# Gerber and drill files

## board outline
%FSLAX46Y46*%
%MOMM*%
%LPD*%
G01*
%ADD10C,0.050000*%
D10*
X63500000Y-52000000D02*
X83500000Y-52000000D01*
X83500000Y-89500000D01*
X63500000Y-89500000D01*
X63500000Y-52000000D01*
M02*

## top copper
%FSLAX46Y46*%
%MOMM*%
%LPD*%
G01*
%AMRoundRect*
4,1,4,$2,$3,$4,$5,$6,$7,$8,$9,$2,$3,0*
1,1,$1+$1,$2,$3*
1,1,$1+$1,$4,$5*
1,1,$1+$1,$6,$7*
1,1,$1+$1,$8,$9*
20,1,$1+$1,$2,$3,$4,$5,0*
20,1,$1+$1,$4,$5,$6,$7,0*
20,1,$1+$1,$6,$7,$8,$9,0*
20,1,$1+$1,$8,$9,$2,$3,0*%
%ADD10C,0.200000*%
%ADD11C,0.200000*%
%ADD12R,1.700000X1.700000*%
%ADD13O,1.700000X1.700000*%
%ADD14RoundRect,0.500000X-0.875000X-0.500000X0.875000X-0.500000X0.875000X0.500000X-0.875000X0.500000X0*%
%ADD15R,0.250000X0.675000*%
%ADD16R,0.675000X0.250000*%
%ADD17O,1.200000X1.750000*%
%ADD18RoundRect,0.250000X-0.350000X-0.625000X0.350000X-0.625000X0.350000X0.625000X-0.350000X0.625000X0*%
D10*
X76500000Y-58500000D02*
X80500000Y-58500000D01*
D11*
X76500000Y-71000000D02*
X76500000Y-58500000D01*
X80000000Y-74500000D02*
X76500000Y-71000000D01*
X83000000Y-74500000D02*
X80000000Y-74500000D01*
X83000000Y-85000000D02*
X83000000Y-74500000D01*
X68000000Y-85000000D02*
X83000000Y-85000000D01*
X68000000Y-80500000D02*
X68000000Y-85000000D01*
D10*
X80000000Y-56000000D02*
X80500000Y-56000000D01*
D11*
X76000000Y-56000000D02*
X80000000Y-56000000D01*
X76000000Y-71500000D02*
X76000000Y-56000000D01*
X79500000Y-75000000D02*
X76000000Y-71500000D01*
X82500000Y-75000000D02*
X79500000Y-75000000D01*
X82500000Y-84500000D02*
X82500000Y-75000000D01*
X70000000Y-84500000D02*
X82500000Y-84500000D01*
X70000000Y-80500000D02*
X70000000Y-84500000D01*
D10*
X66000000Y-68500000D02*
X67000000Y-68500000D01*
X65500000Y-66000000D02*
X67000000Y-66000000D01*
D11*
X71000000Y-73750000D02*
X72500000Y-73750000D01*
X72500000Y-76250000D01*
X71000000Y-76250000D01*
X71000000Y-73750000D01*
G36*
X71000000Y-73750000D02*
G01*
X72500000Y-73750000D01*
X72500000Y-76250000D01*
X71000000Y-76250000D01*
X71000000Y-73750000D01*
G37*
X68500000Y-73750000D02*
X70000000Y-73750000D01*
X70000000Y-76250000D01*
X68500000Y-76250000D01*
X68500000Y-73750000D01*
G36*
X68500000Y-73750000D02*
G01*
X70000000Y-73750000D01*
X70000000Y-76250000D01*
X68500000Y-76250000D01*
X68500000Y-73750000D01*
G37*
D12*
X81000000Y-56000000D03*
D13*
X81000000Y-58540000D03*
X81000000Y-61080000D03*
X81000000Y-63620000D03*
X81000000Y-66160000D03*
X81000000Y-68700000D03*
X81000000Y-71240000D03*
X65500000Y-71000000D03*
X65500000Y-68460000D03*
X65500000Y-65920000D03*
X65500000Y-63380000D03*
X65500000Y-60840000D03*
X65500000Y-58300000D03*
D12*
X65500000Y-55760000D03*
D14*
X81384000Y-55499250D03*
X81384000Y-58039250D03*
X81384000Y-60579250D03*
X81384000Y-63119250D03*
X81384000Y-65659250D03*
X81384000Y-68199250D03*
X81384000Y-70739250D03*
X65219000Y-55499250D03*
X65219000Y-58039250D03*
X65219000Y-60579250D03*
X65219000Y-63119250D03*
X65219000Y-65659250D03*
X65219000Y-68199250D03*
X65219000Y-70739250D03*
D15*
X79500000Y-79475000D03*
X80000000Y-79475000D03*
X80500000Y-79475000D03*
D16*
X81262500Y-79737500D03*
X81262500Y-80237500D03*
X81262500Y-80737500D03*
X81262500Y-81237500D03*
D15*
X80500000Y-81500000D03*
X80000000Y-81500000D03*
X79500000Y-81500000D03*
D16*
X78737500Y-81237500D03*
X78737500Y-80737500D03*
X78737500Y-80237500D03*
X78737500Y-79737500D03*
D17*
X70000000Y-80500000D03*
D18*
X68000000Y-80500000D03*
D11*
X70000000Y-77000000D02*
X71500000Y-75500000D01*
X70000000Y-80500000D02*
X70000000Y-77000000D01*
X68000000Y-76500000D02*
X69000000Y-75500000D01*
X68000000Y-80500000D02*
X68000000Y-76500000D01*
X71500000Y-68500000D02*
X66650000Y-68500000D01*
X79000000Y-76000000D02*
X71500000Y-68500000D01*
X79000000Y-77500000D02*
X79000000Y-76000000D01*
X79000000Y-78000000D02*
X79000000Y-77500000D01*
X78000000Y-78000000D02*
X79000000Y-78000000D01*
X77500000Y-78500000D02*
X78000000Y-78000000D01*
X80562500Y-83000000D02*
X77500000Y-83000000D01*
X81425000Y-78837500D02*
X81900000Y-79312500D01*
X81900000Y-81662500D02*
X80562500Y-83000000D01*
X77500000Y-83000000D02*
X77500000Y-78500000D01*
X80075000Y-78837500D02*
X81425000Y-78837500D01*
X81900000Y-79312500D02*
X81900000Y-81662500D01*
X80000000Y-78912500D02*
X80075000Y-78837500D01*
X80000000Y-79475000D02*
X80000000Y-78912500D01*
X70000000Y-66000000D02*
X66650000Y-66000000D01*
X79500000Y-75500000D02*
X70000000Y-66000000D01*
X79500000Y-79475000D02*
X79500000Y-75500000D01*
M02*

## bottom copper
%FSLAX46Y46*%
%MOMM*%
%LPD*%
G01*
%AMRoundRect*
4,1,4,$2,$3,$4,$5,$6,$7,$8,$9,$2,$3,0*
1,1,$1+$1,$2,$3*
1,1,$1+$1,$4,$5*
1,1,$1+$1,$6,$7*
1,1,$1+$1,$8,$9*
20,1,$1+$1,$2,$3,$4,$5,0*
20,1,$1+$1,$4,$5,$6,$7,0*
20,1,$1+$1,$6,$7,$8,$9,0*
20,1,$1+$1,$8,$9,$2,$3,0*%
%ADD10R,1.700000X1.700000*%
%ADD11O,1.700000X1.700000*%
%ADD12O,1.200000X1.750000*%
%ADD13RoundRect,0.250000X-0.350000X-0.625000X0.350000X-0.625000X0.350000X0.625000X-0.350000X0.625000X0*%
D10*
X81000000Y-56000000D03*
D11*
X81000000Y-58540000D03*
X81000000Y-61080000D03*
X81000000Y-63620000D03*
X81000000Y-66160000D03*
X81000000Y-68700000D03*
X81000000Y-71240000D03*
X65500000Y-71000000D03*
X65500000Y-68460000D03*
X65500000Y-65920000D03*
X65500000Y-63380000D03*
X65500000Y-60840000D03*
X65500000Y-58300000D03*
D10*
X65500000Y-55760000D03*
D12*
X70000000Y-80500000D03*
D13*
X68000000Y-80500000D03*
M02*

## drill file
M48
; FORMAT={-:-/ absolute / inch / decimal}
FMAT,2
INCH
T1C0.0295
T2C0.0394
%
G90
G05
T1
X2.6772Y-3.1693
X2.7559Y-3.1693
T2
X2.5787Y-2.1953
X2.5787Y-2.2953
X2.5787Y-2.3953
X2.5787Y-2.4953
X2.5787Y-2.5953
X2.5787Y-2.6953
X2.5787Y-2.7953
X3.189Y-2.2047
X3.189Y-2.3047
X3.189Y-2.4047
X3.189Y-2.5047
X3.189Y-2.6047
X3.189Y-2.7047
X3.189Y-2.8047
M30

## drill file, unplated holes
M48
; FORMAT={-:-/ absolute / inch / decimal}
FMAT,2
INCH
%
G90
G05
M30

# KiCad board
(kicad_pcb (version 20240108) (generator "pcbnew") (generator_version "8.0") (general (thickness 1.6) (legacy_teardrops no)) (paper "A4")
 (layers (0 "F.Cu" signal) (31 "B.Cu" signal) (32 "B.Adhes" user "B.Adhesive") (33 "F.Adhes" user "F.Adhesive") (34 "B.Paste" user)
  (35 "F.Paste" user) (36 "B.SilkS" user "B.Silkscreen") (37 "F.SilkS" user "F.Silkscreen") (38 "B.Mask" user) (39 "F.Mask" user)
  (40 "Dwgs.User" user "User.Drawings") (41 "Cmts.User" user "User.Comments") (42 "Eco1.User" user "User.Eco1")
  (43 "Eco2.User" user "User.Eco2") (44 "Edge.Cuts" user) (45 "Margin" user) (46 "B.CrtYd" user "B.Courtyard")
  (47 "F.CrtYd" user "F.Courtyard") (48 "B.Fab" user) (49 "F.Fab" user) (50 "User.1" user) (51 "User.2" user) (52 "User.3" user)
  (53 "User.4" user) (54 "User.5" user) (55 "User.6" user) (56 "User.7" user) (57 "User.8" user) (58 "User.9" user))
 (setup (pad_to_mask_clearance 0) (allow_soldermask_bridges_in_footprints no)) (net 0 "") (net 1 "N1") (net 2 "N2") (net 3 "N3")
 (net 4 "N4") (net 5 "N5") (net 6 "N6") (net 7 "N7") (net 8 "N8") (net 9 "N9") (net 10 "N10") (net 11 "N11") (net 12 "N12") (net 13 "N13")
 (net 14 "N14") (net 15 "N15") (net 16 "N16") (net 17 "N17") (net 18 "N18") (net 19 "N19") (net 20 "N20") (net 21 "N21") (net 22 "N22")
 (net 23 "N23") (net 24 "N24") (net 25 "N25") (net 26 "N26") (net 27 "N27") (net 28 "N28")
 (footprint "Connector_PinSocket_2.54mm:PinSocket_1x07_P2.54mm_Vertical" (layer "F.Cu") (at 65.5 55.76)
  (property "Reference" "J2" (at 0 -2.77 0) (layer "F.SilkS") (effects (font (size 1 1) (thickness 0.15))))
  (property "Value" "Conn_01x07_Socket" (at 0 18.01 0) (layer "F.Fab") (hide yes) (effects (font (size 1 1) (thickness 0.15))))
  (pad "1" thru_hole rect (at 0 0) (size 1.7 1.7) (drill 1) (layers "*.Cu" "*.Mask") (remove_unused_layers no) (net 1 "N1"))
  (pad "2" thru_hole oval (at 0 2.54) (size 1.7 1.7) (drill 1) (layers "*.Cu" "*.Mask") (remove_unused_layers no) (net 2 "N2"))
  (pad "3" thru_hole oval (at 0 5.08) (size 1.7 1.7) (drill 1) (layers "*.Cu" "*.Mask") (remove_unused_layers no) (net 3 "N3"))
  (pad "4" thru_hole oval (at 0 7.62) (size 1.7 1.7) (drill 1) (layers "*.Cu" "*.Mask") (remove_unused_layers no) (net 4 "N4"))
  (pad "5" thru_hole oval (at 0 10.16) (size 1.7 1.7) (drill 1) (layers "*.Cu" "*.Mask") (remove_unused_layers no) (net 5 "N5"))
  (pad "6" thru_hole oval (at 0 12.7) (size 1.7 1.7) (drill 1) (layers "*.Cu" "*.Mask") (remove_unused_layers no) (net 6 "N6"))
  (pad "7" thru_hole oval (at 0 15.24) (size 1.7 1.7) (drill 1) (layers "*.Cu" "*.Mask") (remove_unused_layers no) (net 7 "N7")))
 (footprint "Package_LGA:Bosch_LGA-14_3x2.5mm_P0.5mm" (layer "F.Cu") (at 80 80.4875)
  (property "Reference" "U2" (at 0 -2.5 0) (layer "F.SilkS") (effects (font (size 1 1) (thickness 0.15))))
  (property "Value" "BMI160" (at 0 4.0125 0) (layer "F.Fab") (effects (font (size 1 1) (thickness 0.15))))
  (pad "1" smd rect (at -1.2625 -0.75) (size 0.675 0.25) (layers "F.Cu" "F.Paste" "F.Mask") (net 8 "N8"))
  (pad "2" smd rect (at -1.2625 -0.25) (size 0.675 0.25) (layers "F.Cu" "F.Paste" "F.Mask") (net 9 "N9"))
  (pad "3" smd rect (at -1.2625 0.25) (size 0.675 0.25) (layers "F.Cu" "F.Paste" "F.Mask") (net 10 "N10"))
  (pad "4" smd rect (at -1.2625 0.75) (size 0.675 0.25) (layers "F.Cu" "F.Paste" "F.Mask") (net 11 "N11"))
  (pad "5" smd rect (at -0.5 1.0125) (size 0.25 0.675) (layers "F.Cu" "F.Paste" "F.Mask") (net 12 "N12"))
  (pad "6" smd rect (at 0 1.0125) (size 0.25 0.675) (layers "F.Cu" "F.Paste" "F.Mask") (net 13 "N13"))
  (pad "7" smd rect (at 0.5 1.0125) (size 0.25 0.675) (layers "F.Cu" "F.Paste" "F.Mask") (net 13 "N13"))
  (pad "8" smd rect (at 1.2625 0.75) (size 0.675 0.25) (layers "F.Cu" "F.Paste" "F.Mask") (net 12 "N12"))
  (pad "9" smd rect (at 1.2625 0.25) (size 0.675 0.25) (layers "F.Cu" "F.Paste" "F.Mask") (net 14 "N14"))
  (pad "10" smd rect (at 1.2625 -0.25) (size 0.675 0.25) (layers "F.Cu" "F.Paste" "F.Mask") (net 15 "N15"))
  (pad "11" smd rect (at 1.2625 -0.75) (size 0.675 0.25) (layers "F.Cu" "F.Paste" "F.Mask") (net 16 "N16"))
  (pad "12" smd rect (at 0.5 -1.0125) (size 0.25 0.675) (layers "F.Cu" "F.Paste" "F.Mask") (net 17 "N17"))
  (pad "13" smd rect (at 0 -1.0125) (size 0.25 0.675) (layers "F.Cu" "F.Paste" "F.Mask") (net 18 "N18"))
  (pad "14" smd rect (at -0.5 -1.0125) (size 0.25 0.675) (layers "F.Cu" "F.Paste" "F.Mask") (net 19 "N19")))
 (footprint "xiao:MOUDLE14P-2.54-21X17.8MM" (layer "F.Cu") (at 64.384 73.61925)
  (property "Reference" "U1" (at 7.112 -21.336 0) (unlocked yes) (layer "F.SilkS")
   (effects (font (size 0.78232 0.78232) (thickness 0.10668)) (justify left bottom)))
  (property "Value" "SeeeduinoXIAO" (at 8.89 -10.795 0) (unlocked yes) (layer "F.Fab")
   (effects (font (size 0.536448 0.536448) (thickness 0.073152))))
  (pad "1" smd roundrect (at 0.835 -18.12) (size 2.75 2) (layers "F.Cu" "F.Paste" "F.Mask") (roundrect_rratio 0.25) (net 1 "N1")
   (solder_mask_margin 0.1016) (thermal_bridge_angle 0))
  (pad "2" smd roundrect (at 0.835 -15.58) (size 2.75 2) (layers "F.Cu" "F.Paste" "F.Mask") (roundrect_rratio 0.25) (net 2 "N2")
   (solder_mask_margin 0.1016) (thermal_bridge_angle 0))
  (pad "3" smd roundrect (at 0.835 -13.04) (size 2.75 2) (layers "F.Cu" "F.Paste" "F.Mask") (roundrect_rratio 0.25) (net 3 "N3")
   (solder_mask_margin 0.1016) (thermal_bridge_angle 0))
  (pad "4" smd roundrect (at 0.835 -10.5) (size 2.75 2) (layers "F.Cu" "F.Paste" "F.Mask") (roundrect_rratio 0.25) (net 4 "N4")
   (solder_mask_margin 0.1016) (thermal_bridge_angle 0))
  (pad "5" smd roundrect (at 0.835 -7.96) (size 2.75 2) (layers "F.Cu" "F.Paste" "F.Mask") (roundrect_rratio 0.25) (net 5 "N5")
   (solder_mask_margin 0.1016) (thermal_bridge_angle 0))
  (pad "6" smd roundrect (at 0.835 -5.42) (size 2.75 2) (layers "F.Cu" "F.Paste" "F.Mask") (roundrect_rratio 0.25) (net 6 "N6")
   (solder_mask_margin 0.1016) (thermal_bridge_angle 0))
  (pad "7" smd roundrect (at 0.835 -2.88) (size 2.75 2) (layers "F.Cu" "F.Paste" "F.Mask") (roundrect_rratio 0.25) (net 7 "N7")
   (solder_mask_margin 0.1016) (thermal_bridge_angle 0))
  (pad "8" smd roundrect (at 17 -2.88) (size 2.75 2) (layers "F.Cu" "F.Paste" "F.Mask") (roundrect_rratio 0.25) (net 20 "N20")
   (solder_mask_margin 0.1016) (thermal_bridge_angle 0))
  (pad "9" smd roundrect (at 17 -5.42) (size 2.75 2) (layers "F.Cu" "F.Paste" "F.Mask") (roundrect_rratio 0.25) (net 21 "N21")
   (solder_mask_margin 0.1016) (thermal_bridge_angle 0))
  (pad "10" smd roundrect (at 17 -7.96) (size 2.75 2) (layers "F.Cu" "F.Paste" "F.Mask") (roundrect_rratio 0.25) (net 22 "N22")
   (solder_mask_margin 0.1016) (thermal_bridge_angle 0))
  (pad "11" smd roundrect (at 17 -10.5) (size 2.75 2) (layers "F.Cu" "F.Paste" "F.Mask") (roundrect_rratio 0.25) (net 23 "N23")
   (solder_mask_margin 0.1016) (thermal_bridge_angle 0))
  (pad "12" smd roundrect (at 17 -13.04) (size 2.75 2) (layers "F.Cu" "F.Paste" "F.Mask") (roundrect_rratio 0.25) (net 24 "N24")
   (solder_mask_margin 0.1016) (thermal_bridge_angle 0))
  (pad "13" smd roundrect (at 17 -15.58) (size 2.75 2) (layers "F.Cu" "F.Paste" "F.Mask") (roundrect_rratio 0.25) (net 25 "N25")
   (solder_mask_margin 0.1016) (thermal_bridge_angle 0))
  (pad "14" smd roundrect (at 17 -18.12) (size 2.75 2) (layers "F.Cu" "F.Paste" "F.Mask") (roundrect_rratio 0.25) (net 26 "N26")
   (solder_mask_margin 0.1016) (thermal_bridge_angle 0))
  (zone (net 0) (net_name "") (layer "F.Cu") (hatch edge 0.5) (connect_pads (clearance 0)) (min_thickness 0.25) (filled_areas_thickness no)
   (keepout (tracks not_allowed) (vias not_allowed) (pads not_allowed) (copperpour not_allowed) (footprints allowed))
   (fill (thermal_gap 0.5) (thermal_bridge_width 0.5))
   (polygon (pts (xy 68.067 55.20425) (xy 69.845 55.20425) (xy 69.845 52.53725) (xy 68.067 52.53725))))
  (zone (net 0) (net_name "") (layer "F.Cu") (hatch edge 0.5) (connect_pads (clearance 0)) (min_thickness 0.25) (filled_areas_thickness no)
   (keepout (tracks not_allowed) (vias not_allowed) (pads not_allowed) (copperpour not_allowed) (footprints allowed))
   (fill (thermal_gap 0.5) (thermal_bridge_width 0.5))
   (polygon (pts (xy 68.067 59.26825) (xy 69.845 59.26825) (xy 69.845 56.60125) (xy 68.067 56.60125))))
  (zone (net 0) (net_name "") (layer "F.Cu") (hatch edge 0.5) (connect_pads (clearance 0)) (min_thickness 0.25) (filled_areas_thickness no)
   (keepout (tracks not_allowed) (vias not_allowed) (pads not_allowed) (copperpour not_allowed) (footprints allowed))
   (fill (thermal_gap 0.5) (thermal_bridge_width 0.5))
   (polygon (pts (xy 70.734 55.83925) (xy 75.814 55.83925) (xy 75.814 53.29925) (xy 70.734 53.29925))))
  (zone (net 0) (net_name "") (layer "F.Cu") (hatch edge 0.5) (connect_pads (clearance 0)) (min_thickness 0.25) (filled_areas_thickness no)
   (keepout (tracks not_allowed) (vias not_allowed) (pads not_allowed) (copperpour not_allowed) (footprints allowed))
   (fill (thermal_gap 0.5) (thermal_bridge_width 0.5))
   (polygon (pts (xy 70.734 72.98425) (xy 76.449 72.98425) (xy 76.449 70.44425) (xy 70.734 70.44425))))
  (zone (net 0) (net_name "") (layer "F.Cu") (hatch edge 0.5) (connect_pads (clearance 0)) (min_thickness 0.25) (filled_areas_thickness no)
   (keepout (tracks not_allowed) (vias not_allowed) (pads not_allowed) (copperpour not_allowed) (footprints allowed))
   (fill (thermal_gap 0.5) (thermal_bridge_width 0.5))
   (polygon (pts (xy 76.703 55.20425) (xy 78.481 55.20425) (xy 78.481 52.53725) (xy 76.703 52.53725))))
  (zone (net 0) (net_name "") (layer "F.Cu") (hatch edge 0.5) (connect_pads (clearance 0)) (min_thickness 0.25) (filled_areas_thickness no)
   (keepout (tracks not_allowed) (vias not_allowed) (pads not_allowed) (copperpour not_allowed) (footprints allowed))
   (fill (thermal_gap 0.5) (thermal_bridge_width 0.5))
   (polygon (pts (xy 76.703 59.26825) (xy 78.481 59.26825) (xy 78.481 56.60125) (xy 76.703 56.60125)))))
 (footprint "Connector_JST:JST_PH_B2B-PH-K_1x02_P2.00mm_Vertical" (layer "F.Cu") (at 68 80.5)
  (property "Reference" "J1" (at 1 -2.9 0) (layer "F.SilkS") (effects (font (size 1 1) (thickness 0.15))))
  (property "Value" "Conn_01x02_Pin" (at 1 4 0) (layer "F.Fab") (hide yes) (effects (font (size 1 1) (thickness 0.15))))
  (pad "1" thru_hole roundrect (at 0 0) (size 1.2 1.75) (drill 0.75) (layers "*.Cu" "*.Mask") (remove_unused_layers no)
   (roundrect_rratio 0.208333) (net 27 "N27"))
  (pad "2" thru_hole oval (at 2 0) (size 1.2 1.75) (drill 0.75) (layers "*.Cu" "*.Mask") (remove_unused_layers no) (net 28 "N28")))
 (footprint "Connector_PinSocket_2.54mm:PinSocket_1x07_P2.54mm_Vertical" (layer "F.Cu") (at 81 56)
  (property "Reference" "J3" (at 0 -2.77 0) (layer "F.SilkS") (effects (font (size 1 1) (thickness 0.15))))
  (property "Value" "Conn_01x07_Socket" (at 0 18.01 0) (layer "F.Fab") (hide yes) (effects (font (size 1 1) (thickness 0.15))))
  (pad "1" thru_hole rect (at 0 0) (size 1.7 1.7) (drill 1) (layers "*.Cu" "*.Mask") (remove_unused_layers no) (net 26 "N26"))
  (pad "2" thru_hole oval (at 0 2.54) (size 1.7 1.7) (drill 1) (layers "*.Cu" "*.Mask") (remove_unused_layers no) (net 25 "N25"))
  (pad "3" thru_hole oval (at 0 5.08) (size 1.7 1.7) (drill 1) (layers "*.Cu" "*.Mask") (remove_unused_layers no) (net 24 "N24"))
  (pad "4" thru_hole oval (at 0 7.62) (size 1.7 1.7) (drill 1) (layers "*.Cu" "*.Mask") (remove_unused_layers no) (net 23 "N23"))
  (pad "5" thru_hole oval (at 0 10.16) (size 1.7 1.7) (drill 1) (layers "*.Cu" "*.Mask") (remove_unused_layers no) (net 22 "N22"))
  (pad "6" thru_hole oval (at 0 12.7) (size 1.7 1.7) (drill 1) (layers "*.Cu" "*.Mask") (remove_unused_layers no) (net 21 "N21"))
  (pad "7" thru_hole oval (at 0 15.24) (size 1.7 1.7) (drill 1) (layers "*.Cu" "*.Mask") (remove_unused_layers no) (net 20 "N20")))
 (gr_line (start 80 56) (end 80.5 56) (stroke (width 0.2) (type default)) (layer "F.Cu"))
 (gr_line (start 83 85) (end 83 74.5) (stroke (width 0.2) (type default)) (layer "F.Cu") (net 27))
 (gr_line (start 83 74.5) (end 80 74.5) (stroke (width 0.2) (type default)) (layer "F.Cu") (net 27))
 (gr_line (start 68 85) (end 83 85) (stroke (width 0.2) (type default)) (layer "F.Cu") (net 27))
 (gr_rect (start 68.5 73.75) (end 70 76.25) (stroke (width 0.2) (type solid)) (fill solid) (layer "F.Cu") (net 27))
 (gr_line (start 76.5 71) (end 76.5 58.5) (stroke (width 0.2) (type default)) (layer "F.Cu") (net 27))
 (gr_line (start 76 71.5) (end 76 56) (stroke (width 0.2) (type default)) (layer "F.Cu") (net 28))
 (gr_line (start 65.5 66) (end 67 66) (stroke (width 0.2) (type default)) (layer "F.Cu"))
 (gr_line (start 76 56) (end 80 56) (stroke (width 0.2) (type default)) (layer "F.Cu") (net 28))
 (gr_line (start 82.5 84.5) (end 82.5 75) (stroke (width 0.2) (type default)) (layer "F.Cu") (net 28))
 (gr_line (start 70 80.5) (end 70 84.5) (stroke (width 0.2) (type default)) (layer "F.Cu") (net 28))
 (gr_line (start 80 74.5) (end 76.5 71) (stroke (width 0.2) (type default)) (layer "F.Cu") (net 27))
 (gr_line (start 82.5 75) (end 79.5 75) (stroke (width 0.2) (type default)) (layer "F.Cu") (net 28))
 (gr_line (start 68 80.5) (end 68 85) (stroke (width 0.2) (type default)) (layer "F.Cu") (net 27))
 (gr_line (start 79.5 75) (end 76 71.5) (stroke (width 0.2) (type default)) (layer "F.Cu") (net 28))
 (gr_line (start 66 68.5) (end 67 68.5) (stroke (width 0.2) (type default)) (layer "F.Cu"))
 (gr_line (start 70 84.5) (end 82.5 84.5) (stroke (width 0.2) (type default)) (layer "F.Cu") (net 28))
 (gr_line (start 76.5 58.5) (end 80.5 58.5) (stroke (width 0.2) (type default)) (layer "F.Cu"))
 (gr_rect (start 71 73.75) (end 72.5 76.25) (stroke (width 0.2) (type solid)) (fill solid) (layer "F.Cu") (net 28))
 (gr_rect (start 63.5 52) (end 83.5 89.5) (stroke (width 0.05) (type default)) (fill none) (layer "Edge.Cuts"))
 (segment (start 70 80.5) (end 70 77) (width 0.2) (layer "F.Cu") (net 28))
 (segment (start 70 77) (end 71.5 75.5) (width 0.2) (layer "F.Cu") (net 28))
 (segment (start 68 80.5) (end 68 76.5) (width 0.2) (layer "F.Cu") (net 27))
 (segment (start 68 76.5) (end 69 75.5) (width 0.2) (layer "F.Cu") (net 27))
 (segment (start 70 66) (end 66.65 66) (width 0.2) (layer "F.Cu") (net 19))
 (segment (start 79.5 79.475) (end 79.5 75.5) (width 0.2) (layer "F.Cu") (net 19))
 (segment (start 79.5 75.5) (end 70 66) (width 0.2) (layer "F.Cu") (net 19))
 (segment (start 81.425 78.8375) (end 81.9 79.3125) (width 0.2) (layer "F.Cu") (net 18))
 (segment (start 78 78) (end 79 78) (width 0.2) (layer "F.Cu") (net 18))
 (segment (start 80.075 78.8375) (end 81.425 78.8375) (width 0.2) (layer "F.Cu") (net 18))
 (segment (start 79 77.5) (end 79 76) (width 0.2) (layer "F.Cu") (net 18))
 (segment (start 79 76) (end 71.5 68.5) (width 0.2) (layer "F.Cu") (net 18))
 (segment (start 80 79.475) (end 80 78.9125) (width 0.2) (layer "F.Cu") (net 18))
 (segment (start 77.5 78.5) (end 78 78) (width 0.2) (layer "F.Cu") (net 18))
 (segment (start 71.5 68.5) (end 66.65 68.5) (width 0.2) (layer "F.Cu") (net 18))
 (segment (start 77.5 83) (end 77.5 78.5) (width 0.2) (layer "F.Cu") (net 18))
 (segment (start 81.9 79.3125) (end 81.9 81.6625) (width 0.2) (layer "F.Cu") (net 18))
 (segment (start 79 78) (end 79 77.5) (width 0.2) (layer "F.Cu") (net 18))
 (segment (start 81.9 81.6625) (end 80.5625 83) (width 0.2) (layer "F.Cu") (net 18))
 (segment (start 80 78.9125) (end 80.075 78.8375) (width 0.2) (layer "F.Cu") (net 18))
 (segment (start 80.5625 83) (end 77.5 83) (width 0.2) (layer "F.Cu") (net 18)))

